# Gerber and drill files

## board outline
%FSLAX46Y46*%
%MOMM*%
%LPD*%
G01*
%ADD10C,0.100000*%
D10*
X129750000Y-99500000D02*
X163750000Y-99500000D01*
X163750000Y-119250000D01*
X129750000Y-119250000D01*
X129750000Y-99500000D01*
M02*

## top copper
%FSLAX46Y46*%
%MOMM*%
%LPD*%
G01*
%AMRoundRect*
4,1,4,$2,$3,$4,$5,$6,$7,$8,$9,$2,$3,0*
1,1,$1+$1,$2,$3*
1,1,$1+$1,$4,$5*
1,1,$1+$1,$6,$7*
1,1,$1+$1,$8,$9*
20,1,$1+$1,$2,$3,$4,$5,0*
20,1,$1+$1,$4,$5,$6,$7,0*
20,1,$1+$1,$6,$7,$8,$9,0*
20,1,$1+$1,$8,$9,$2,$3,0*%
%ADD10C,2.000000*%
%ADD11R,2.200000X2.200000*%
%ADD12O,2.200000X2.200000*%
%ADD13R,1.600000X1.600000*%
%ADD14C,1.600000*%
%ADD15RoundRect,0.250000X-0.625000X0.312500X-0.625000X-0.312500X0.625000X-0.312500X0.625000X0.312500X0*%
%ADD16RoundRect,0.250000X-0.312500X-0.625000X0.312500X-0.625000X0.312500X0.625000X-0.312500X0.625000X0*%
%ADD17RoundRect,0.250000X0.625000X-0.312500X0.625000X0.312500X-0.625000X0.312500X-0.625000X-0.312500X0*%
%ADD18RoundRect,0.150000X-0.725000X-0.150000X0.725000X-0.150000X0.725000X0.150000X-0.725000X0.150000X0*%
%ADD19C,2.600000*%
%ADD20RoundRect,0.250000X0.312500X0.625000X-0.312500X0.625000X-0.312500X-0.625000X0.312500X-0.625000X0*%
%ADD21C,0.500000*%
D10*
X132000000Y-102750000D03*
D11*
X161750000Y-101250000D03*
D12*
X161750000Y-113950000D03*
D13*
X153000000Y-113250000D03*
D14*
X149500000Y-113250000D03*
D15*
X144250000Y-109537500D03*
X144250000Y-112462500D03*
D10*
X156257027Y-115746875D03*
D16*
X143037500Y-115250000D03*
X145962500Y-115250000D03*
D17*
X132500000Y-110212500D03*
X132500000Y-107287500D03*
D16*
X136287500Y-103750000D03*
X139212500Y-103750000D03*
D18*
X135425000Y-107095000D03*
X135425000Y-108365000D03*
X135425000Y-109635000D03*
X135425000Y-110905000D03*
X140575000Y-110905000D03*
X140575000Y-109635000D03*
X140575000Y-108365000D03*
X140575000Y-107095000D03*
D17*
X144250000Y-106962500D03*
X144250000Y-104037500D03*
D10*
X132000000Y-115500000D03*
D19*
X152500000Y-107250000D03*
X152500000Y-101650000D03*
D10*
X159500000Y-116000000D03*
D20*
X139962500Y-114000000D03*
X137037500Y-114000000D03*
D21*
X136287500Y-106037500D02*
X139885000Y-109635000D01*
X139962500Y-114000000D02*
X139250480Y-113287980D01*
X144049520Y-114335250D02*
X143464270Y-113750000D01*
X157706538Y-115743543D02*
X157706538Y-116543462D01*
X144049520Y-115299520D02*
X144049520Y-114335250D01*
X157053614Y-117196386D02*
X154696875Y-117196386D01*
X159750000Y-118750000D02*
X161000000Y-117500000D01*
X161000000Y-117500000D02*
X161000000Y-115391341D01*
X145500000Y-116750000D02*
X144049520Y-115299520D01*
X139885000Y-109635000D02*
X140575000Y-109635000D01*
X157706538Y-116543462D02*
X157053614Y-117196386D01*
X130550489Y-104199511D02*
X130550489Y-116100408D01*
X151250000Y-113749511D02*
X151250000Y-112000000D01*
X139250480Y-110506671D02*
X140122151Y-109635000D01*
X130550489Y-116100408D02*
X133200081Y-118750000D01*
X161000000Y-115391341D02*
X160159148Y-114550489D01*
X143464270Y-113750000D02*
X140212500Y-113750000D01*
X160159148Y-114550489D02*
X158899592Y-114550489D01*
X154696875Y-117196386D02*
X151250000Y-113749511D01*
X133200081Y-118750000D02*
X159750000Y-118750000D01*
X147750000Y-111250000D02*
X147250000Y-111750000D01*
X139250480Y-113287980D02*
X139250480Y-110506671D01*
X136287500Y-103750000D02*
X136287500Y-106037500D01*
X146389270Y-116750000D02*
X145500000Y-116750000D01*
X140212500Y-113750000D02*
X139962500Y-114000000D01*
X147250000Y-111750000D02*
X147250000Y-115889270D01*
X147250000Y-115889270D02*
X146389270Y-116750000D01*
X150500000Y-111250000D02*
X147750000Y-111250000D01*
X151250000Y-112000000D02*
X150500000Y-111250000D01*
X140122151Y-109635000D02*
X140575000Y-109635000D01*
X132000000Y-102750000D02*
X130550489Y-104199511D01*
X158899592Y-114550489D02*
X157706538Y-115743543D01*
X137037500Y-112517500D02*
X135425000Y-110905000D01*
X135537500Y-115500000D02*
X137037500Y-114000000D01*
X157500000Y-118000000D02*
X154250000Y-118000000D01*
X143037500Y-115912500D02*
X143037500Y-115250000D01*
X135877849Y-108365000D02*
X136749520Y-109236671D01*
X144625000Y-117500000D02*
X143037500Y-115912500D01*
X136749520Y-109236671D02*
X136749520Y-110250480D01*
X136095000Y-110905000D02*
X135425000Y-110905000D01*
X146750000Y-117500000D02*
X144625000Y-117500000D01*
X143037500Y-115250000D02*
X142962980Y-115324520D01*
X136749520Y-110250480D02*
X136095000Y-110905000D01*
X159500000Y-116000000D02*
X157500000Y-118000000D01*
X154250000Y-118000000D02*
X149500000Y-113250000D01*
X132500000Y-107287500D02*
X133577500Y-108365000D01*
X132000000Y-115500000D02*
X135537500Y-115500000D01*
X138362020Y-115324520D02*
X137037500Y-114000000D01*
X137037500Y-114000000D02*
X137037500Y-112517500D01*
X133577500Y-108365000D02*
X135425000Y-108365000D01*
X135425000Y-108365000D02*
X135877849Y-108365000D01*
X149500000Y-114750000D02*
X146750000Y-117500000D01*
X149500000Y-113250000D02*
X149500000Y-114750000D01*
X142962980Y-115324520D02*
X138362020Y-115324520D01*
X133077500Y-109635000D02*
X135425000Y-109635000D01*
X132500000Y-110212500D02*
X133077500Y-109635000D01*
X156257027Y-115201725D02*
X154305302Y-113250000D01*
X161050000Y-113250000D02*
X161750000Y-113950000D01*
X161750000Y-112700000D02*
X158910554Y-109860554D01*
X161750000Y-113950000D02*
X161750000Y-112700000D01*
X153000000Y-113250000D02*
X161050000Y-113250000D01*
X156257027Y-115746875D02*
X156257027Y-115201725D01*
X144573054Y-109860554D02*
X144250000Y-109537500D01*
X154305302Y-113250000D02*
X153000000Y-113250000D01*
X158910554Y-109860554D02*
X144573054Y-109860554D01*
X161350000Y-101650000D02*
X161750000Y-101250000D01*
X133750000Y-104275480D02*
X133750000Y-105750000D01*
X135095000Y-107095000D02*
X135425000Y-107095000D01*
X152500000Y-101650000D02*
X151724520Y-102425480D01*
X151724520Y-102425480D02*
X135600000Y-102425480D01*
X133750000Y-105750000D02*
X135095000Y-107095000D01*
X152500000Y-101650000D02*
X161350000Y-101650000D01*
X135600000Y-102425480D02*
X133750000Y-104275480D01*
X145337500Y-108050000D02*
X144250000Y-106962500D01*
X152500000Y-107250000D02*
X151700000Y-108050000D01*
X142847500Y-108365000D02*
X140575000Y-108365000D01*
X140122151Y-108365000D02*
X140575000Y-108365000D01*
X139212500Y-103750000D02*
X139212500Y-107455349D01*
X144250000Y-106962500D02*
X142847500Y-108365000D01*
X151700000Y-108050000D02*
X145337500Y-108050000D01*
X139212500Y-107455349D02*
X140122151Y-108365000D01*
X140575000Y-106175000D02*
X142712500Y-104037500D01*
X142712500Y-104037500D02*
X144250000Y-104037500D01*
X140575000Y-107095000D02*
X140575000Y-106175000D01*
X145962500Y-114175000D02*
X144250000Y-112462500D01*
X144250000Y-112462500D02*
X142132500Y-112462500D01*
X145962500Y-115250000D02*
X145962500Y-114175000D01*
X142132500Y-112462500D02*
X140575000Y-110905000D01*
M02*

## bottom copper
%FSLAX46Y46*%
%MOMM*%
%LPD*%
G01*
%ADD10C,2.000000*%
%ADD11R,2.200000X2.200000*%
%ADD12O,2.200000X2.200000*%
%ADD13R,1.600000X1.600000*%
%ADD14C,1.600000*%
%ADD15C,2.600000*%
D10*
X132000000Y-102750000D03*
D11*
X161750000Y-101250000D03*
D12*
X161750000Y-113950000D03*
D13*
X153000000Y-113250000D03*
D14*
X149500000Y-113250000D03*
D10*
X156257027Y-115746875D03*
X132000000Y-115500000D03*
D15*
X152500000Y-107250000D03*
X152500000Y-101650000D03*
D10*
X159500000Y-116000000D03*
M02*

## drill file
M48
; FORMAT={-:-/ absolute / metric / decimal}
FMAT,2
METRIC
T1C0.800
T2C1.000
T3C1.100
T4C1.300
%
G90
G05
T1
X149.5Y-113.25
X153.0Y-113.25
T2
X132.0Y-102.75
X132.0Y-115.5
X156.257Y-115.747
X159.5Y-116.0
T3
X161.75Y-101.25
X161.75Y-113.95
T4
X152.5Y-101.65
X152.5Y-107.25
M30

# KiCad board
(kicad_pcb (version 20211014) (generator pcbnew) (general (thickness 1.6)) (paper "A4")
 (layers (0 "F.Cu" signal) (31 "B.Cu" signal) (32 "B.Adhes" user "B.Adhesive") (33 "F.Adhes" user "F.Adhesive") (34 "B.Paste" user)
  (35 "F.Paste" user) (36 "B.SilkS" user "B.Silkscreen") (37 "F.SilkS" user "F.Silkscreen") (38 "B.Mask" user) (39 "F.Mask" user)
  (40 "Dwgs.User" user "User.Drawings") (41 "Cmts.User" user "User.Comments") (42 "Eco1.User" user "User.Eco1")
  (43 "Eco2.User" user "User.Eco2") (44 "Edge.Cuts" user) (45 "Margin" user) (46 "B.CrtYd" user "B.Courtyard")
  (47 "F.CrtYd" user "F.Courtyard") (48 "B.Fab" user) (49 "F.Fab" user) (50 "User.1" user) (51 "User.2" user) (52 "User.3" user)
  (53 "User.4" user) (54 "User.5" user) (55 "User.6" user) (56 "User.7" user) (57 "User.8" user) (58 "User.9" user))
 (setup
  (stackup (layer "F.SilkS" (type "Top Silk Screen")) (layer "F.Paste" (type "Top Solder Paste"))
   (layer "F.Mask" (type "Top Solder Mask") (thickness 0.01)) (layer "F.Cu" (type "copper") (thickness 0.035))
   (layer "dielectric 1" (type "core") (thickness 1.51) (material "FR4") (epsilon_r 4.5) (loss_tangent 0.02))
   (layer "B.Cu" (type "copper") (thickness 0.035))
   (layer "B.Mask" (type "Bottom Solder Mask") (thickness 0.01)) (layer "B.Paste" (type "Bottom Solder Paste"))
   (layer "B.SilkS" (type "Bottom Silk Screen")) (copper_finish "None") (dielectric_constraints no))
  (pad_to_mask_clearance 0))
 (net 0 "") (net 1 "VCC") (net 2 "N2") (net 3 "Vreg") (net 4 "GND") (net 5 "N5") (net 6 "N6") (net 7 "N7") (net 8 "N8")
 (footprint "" (layer "F.Cu") (at 132 102.75)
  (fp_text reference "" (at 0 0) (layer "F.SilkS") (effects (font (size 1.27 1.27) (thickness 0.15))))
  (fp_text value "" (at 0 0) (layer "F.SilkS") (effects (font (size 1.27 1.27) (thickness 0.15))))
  (pad "1" thru_hole circle (at 0 0) (size 2 2) (drill 1) (layers *.Cu *.Mask) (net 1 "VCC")))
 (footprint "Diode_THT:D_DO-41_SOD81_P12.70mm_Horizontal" (layer "F.Cu") (at 161.75 101.25 -90)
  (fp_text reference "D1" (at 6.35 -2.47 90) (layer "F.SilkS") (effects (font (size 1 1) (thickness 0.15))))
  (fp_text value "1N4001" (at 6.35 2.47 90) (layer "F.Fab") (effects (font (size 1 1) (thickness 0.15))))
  (pad "1" thru_hole rect (at 0 0 270) (size 2.2 2.2) (drill 1.1) (layers *.Cu *.Mask) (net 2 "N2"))
  (pad "2" thru_hole oval (at 12.7 0 270) (size 2.2 2.2) (drill 1.1) (layers *.Cu *.Mask) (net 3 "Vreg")))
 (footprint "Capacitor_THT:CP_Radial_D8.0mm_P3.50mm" (layer "F.Cu") (at 153 113.25 180)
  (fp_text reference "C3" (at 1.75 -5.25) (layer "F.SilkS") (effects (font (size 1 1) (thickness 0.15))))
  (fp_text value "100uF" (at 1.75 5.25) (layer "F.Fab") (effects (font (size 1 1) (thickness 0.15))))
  (pad "1" thru_hole rect (at 0 0 180) (size 1.6 1.6) (drill 0.8) (layers *.Cu *.Mask) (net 3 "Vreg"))
  (pad "2" thru_hole circle (at 3.5 0 180) (size 1.6 1.6) (drill 0.8) (layers *.Cu *.Mask) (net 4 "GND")))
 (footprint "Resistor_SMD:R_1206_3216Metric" (layer "F.Cu") (at 144.25 111 -90)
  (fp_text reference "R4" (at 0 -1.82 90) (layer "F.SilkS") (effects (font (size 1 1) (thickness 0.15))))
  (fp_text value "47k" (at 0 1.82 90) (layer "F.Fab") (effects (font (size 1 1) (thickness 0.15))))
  (pad "1" smd roundrect (at -1.4625 0 270) (size 1.125 1.75) (layers "F.Cu" "F.Paste" "F.Mask") (roundrect_rratio 0.2222222222)
   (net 3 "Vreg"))
  (pad "2" smd roundrect (at 1.4625 0 270) (size 1.125 1.75) (layers "F.Cu" "F.Paste" "F.Mask") (roundrect_rratio 0.2222222222) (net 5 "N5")))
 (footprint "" (layer "F.Cu") (at 156.257027 115.746875)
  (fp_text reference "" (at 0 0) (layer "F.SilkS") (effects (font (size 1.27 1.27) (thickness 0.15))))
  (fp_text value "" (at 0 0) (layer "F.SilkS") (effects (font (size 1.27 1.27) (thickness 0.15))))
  (pad "1" thru_hole circle (at 0 0) (size 2 2) (drill 1) (layers *.Cu *.Mask) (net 3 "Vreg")))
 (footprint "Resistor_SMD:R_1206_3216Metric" (layer "F.Cu") (at 144.5 115.25)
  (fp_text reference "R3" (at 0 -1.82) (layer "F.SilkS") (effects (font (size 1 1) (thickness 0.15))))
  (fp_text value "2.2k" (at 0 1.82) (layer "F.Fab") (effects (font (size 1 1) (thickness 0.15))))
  (pad "1" smd roundrect (at -1.4625 0) (size 1.125 1.75) (layers "F.Cu" "F.Paste" "F.Mask") (roundrect_rratio 0.2222222222) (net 4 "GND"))
  (pad "2" smd roundrect (at 1.4625 0) (size 1.125 1.75) (layers "F.Cu" "F.Paste" "F.Mask") (roundrect_rratio 0.2222222222) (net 5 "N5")))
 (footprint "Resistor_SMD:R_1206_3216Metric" (layer "F.Cu") (at 132.5 108.75 90)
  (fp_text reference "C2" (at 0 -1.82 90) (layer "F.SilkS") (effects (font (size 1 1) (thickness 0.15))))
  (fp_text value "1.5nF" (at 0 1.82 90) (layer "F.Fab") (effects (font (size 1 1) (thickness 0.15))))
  (pad "1" smd roundrect (at -1.4625 0 90) (size 1.125 1.75) (layers "F.Cu" "F.Paste" "F.Mask") (roundrect_rratio 0.2222222222) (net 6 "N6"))
  (pad "2" smd roundrect (at 1.4625 0 90) (size 1.125 1.75) (layers "F.Cu" "F.Paste" "F.Mask") (roundrect_rratio 0.2222222222) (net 4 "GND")))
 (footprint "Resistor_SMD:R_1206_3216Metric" (layer "F.Cu") (at 137.75 103.75)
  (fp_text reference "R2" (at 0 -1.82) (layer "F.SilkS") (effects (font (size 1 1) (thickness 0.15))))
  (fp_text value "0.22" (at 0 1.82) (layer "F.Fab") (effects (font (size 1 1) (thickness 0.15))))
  (pad "1" smd roundrect (at -1.4625 0) (size 1.125 1.75) (layers "F.Cu" "F.Paste" "F.Mask") (roundrect_rratio 0.2222222222) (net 1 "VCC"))
  (pad "2" smd roundrect (at 1.4625 0) (size 1.125 1.75) (layers "F.Cu" "F.Paste" "F.Mask") (roundrect_rratio 0.2222222222) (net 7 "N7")))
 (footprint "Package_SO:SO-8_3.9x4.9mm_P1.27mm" (layer "F.Cu") (at 138 109)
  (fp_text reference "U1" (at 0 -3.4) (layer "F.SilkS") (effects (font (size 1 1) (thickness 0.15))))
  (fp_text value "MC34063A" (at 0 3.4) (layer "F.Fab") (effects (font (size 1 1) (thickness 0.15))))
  (pad "1" smd roundrect (at -2.575 -1.905) (size 1.75 0.6) (layers "F.Cu" "F.Paste" "F.Mask") (roundrect_rratio 0.25) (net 2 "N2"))
  (pad "2" smd roundrect (at -2.575 -0.635) (size 1.75 0.6) (layers "F.Cu" "F.Paste" "F.Mask") (roundrect_rratio 0.25) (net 4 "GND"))
  (pad "3" smd roundrect (at -2.575 0.635) (size 1.75 0.6) (layers "F.Cu" "F.Paste" "F.Mask") (roundrect_rratio 0.25) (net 6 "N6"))
  (pad "4" smd roundrect (at -2.575 1.905) (size 1.75 0.6) (layers "F.Cu" "F.Paste" "F.Mask") (roundrect_rratio 0.25) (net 4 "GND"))
  (pad "5" smd roundrect (at 2.575 1.905) (size 1.75 0.6) (layers "F.Cu" "F.Paste" "F.Mask") (roundrect_rratio 0.25) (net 5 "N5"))
  (pad "6" smd roundrect (at 2.575 0.635) (size 1.75 0.6) (layers "F.Cu" "F.Paste" "F.Mask") (roundrect_rratio 0.25) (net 1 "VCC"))
  (pad "7" smd roundrect (at 2.575 -0.635) (size 1.75 0.6) (layers "F.Cu" "F.Paste" "F.Mask") (roundrect_rratio 0.25) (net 7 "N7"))
  (pad "8" smd roundrect (at 2.575 -1.905) (size 1.75 0.6) (layers "F.Cu" "F.Paste" "F.Mask") (roundrect_rratio 0.25) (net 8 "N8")))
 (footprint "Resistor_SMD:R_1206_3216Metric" (layer "F.Cu") (at 144.25 105.5 90)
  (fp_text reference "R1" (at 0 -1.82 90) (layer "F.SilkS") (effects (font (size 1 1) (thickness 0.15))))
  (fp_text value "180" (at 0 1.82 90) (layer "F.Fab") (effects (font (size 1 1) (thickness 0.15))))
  (pad "1" smd roundrect (at -1.4625 0 90) (size 1.125 1.75) (layers "F.Cu" "F.Paste" "F.Mask") (roundrect_rratio 0.2222222222) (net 7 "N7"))
  (pad "2" smd roundrect (at 1.4625 0 90) (size 1.125 1.75) (layers "F.Cu" "F.Paste" "F.Mask") (roundrect_rratio 0.2222222222) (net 8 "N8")))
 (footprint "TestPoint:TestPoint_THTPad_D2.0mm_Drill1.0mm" (layer "F.Cu") (at 132 115.5)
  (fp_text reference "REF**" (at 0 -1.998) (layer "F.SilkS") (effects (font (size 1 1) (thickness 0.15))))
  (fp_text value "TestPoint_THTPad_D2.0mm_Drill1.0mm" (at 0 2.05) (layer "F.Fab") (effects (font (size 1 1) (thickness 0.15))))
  (pad "1" thru_hole circle (at 0 0) (size 2 2) (drill 1) (layers *.Cu *.Mask) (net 4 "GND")))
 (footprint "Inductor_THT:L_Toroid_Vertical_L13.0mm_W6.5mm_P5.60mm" (layer "F.Cu") (at 152.5 107.25 180)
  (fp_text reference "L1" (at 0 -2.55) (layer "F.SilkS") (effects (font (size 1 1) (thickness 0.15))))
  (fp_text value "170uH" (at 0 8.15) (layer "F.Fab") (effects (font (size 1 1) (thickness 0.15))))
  (pad "1" thru_hole circle (at 0 0 180) (size 2.6 2.6) (drill 1.3) (layers *.Cu *.Mask) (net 7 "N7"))
  (pad "2" thru_hole circle (at 0 5.6 180) (size 2.6 2.6) (drill 1.3) (layers *.Cu *.Mask) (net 2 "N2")))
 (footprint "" (layer "F.Cu") (at 159.5 116)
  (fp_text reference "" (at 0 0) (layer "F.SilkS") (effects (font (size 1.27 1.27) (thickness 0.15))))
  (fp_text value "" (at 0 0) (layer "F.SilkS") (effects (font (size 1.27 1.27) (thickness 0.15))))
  (pad "1" thru_hole circle (at 0 0) (size 2 2) (drill 1) (layers *.Cu *.Mask) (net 4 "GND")))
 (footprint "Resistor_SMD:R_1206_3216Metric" (layer "F.Cu") (at 138.5 114 180)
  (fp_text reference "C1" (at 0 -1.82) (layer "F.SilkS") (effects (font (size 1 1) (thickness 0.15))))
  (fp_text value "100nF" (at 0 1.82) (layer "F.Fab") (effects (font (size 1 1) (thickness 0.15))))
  (pad "1" smd roundrect (at -1.4625 0 180) (size 1.125 1.75) (layers "F.Cu" "F.Paste" "F.Mask") (roundrect_rratio 0.2222222222)
   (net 1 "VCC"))
  (pad "2" smd roundrect (at 1.4625 0 180) (size 1.125 1.75) (layers "F.Cu" "F.Paste" "F.Mask") (roundrect_rratio 0.2222222222)
   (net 4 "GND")))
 (gr_rect (start 129.75 99.5) (end 163.75 119.25) (layer "Edge.Cuts") (width 0.1) (fill none))
 (segment (start 136.2875 106.0375) (end 139.885 109.635) (width 0.5) (layer "F.Cu") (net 1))
 (segment (start 139.9625 114) (end 139.25048 113.28798) (width 0.5) (layer "F.Cu") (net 1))
 (segment (start 144.04952 114.33525) (end 143.46427 113.75) (width 0.5) (layer "F.Cu") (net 1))
 (segment (start 157.706538 115.743543) (end 157.706538 116.543462) (width 0.5) (layer "F.Cu") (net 1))
 (segment (start 144.04952 115.29952) (end 144.04952 114.33525) (width 0.5) (layer "F.Cu") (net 1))
 (segment (start 157.053614 117.196386) (end 154.696875 117.196386) (width 0.5) (layer "F.Cu") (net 1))
 (segment (start 159.75 118.75) (end 161 117.5) (width 0.5) (layer "F.Cu") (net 1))
 (segment (start 161 117.5) (end 161 115.391341) (width 0.5) (layer "F.Cu") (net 1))
 (segment (start 145.5 116.75) (end 144.04952 115.29952) (width 0.5) (layer "F.Cu") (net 1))
 (segment (start 139.885 109.635) (end 140.575 109.635) (width 0.5) (layer "F.Cu") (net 1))
 (segment (start 157.706538 116.543462) (end 157.053614 117.196386) (width 0.5) (layer "F.Cu") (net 1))
 (segment (start 130.550489 104.199511) (end 130.550489 116.100408) (width 0.5) (layer "F.Cu") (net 1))
 (segment (start 151.25 113.749511) (end 151.25 112) (width 0.5) (layer "F.Cu") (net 1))
 (segment (start 139.25048 110.506671) (end 140.122151 109.635) (width 0.5) (layer "F.Cu") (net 1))
 (segment (start 130.550489 116.100408) (end 133.200081 118.75) (width 0.5) (layer "F.Cu") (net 1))
 (segment (start 161 115.391341) (end 160.159148 114.550489) (width 0.5) (layer "F.Cu") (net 1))
 (segment (start 143.46427 113.75) (end 140.2125 113.75) (width 0.5) (layer "F.Cu") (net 1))
 (segment (start 160.159148 114.550489) (end 158.899592 114.550489) (width 0.5) (layer "F.Cu") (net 1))
 (segment (start 154.696875 117.196386) (end 151.25 113.749511) (width 0.5) (layer "F.Cu") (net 1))
 (segment (start 133.200081 118.75) (end 159.75 118.75) (width 0.5) (layer "F.Cu") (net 1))
 (segment (start 147.75 111.25) (end 147.25 111.75) (width 0.5) (layer "F.Cu") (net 1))
 (segment (start 139.25048 113.28798) (end 139.25048 110.506671) (width 0.5) (layer "F.Cu") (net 1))
 (segment (start 136.2875 103.75) (end 136.2875 106.0375) (width 0.5) (layer "F.Cu") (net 1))
 (segment (start 146.38927 116.75) (end 145.5 116.75) (width 0.5) (layer "F.Cu") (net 1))
 (segment (start 140.2125 113.75) (end 139.9625 114) (width 0.5) (layer "F.Cu") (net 1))
 (segment (start 147.25 111.75) (end 147.25 115.88927) (width 0.5) (layer "F.Cu") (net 1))
 (segment (start 147.25 115.88927) (end 146.38927 116.75) (width 0.5) (layer "F.Cu") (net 1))
 (segment (start 150.5 111.25) (end 147.75 111.25) (width 0.5) (layer "F.Cu") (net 1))
 (segment (start 151.25 112) (end 150.5 111.25) (width 0.5) (layer "F.Cu") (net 1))
 (segment (start 140.122151 109.635) (end 140.575 109.635) (width 0.5) (layer "F.Cu") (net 1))
 (segment (start 132 102.75) (end 130.550489 104.199511) (width 0.5) (layer "F.Cu") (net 1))
 (segment (start 158.899592 114.550489) (end 157.706538 115.743543) (width 0.5) (layer "F.Cu") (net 1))
 (segment (start 137.0375 112.5175) (end 135.425 110.905) (width 0.5) (layer "F.Cu") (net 4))
 (segment (start 135.5375 115.5) (end 137.0375 114) (width 0.5) (layer "F.Cu") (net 4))
 (segment (start 157.5 118) (end 154.25 118) (width 0.5) (layer "F.Cu") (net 4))
 (segment (start 143.0375 115.9125) (end 143.0375 115.25) (width 0.5) (layer "F.Cu") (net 4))
 (segment (start 135.877849 108.365) (end 136.74952 109.236671) (width 0.5) (layer "F.Cu") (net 4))
 (segment (start 144.625 117.5) (end 143.0375 115.9125) (width 0.5) (layer "F.Cu") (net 4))
 (segment (start 136.74952 109.236671) (end 136.74952 110.25048) (width 0.5) (layer "F.Cu") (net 4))
 (segment (start 136.095 110.905) (end 135.425 110.905) (width 0.5) (layer "F.Cu") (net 4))
 (segment (start 146.75 117.5) (end 144.625 117.5) (width 0.5) (layer "F.Cu") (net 4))
 (segment (start 143.0375 115.25) (end 142.96298 115.32452) (width 0.5) (layer "F.Cu") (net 4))
 (segment (start 136.74952 110.25048) (end 136.095 110.905) (width 0.5) (layer "F.Cu") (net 4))
 (segment (start 159.5 116) (end 157.5 118) (width 0.5) (layer "F.Cu") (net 4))
 (segment (start 154.25 118) (end 149.5 113.25) (width 0.5) (layer "F.Cu") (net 4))
 (segment (start 132.5 107.2875) (end 133.5775 108.365) (width 0.5) (layer "F.Cu") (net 4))
 (segment (start 132 115.5) (end 135.5375 115.5) (width 0.5) (layer "F.Cu") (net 4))
 (segment (start 138.36202 115.32452) (end 137.0375 114) (width 0.5) (layer "F.Cu") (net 4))
 (segment (start 137.0375 114) (end 137.0375 112.5175) (width 0.5) (layer "F.Cu") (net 4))
 (segment (start 133.5775 108.365) (end 135.425 108.365) (width 0.5) (layer "F.Cu") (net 4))
 (segment (start 135.425 108.365) (end 135.877849 108.365) (width 0.5) (layer "F.Cu") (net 4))
 (segment (start 149.5 114.75) (end 146.75 117.5) (width 0.5) (layer "F.Cu") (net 4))
 (segment (start 149.5 113.25) (end 149.5 114.75) (width 0.5) (layer "F.Cu") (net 4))
 (segment (start 142.96298 115.32452) (end 138.36202 115.32452) (width 0.5) (layer "F.Cu") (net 4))
 (segment (start 133.0775 109.635) (end 135.425 109.635) (width 0.5) (layer "F.Cu") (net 6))
 (segment (start 132.5 110.2125) (end 133.0775 109.635) (width 0.5) (layer "F.Cu") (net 6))
 (segment (start 156.257027 115.201725) (end 154.305302 113.25) (width 0.5) (layer "F.Cu") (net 3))
 (segment (start 161.05 113.25) (end 161.75 113.95) (width 0.5) (layer "F.Cu") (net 3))
 (segment (start 161.75 112.7) (end 158.910554 109.860554) (width 0.5) (layer "F.Cu") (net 3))
 (segment (start 161.75 113.95) (end 161.75 112.7) (width 0.5) (layer "F.Cu") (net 3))
 (segment (start 153 113.25) (end 161.05 113.25) (width 0.5) (layer "F.Cu") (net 3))
 (segment (start 156.257027 115.746875) (end 156.257027 115.201725) (width 0.5) (layer "F.Cu") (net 3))
 (segment (start 144.573054 109.860554) (end 144.25 109.5375) (width 0.5) (layer "F.Cu") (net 3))
 (segment (start 154.305302 113.25) (end 153 113.25) (width 0.5) (layer "F.Cu") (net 3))
 (segment (start 158.910554 109.860554) (end 144.573054 109.860554) (width 0.5) (layer "F.Cu") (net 3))
 (segment (start 161.35 101.65) (end 161.75 101.25) (width 0.5) (layer "F.Cu") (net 2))
 (segment (start 133.75 104.27548) (end 133.75 105.75) (width 0.5) (layer "F.Cu") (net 2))
 (segment (start 135.095 107.095) (end 135.425 107.095) (width 0.5) (layer "F.Cu") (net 2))
 (segment (start 152.5 101.65) (end 151.72452 102.42548) (width 0.5) (layer "F.Cu") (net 2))
 (segment (start 151.72452 102.42548) (end 135.6 102.42548) (width 0.5) (layer "F.Cu") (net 2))
 (segment (start 133.75 105.75) (end 135.095 107.095) (width 0.5) (layer "F.Cu") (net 2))
 (segment (start 152.5 101.65) (end 161.35 101.65) (width 0.5) (layer "F.Cu") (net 2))
 (segment (start 135.6 102.42548) (end 133.75 104.27548) (width 0.5) (layer "F.Cu") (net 2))
 (segment (start 145.3375 108.05) (end 144.25 106.9625) (width 0.5) (layer "F.Cu") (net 7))
 (segment (start 152.5 107.25) (end 151.7 108.05) (width 0.5) (layer "F.Cu") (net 7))
 (segment (start 142.8475 108.365) (end 140.575 108.365) (width 0.5) (layer "F.Cu") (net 7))
 (segment (start 140.122151 108.365) (end 140.575 108.365) (width 0.5) (layer "F.Cu") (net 7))
 (segment (start 139.2125 103.75) (end 139.2125 107.455349) (width 0.5) (layer "F.Cu") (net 7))
 (segment (start 144.25 106.9625) (end 142.8475 108.365) (width 0.5) (layer "F.Cu") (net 7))
 (segment (start 151.7 108.05) (end 145.3375 108.05) (width 0.5) (layer "F.Cu") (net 7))
 (segment (start 139.2125 107.455349) (end 140.122151 108.365) (width 0.5) (layer "F.Cu") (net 7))
 (segment (start 140.575 106.175) (end 142.7125 104.0375) (width 0.5) (layer "F.Cu") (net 8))
 (segment (start 142.7125 104.0375) (end 144.25 104.0375) (width 0.5) (layer "F.Cu") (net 8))
 (segment (start 140.575 107.095) (end 140.575 106.175) (width 0.5) (layer "F.Cu") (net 8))
 (segment (start 145.9625 114.175) (end 144.25 112.4625) (width 0.5) (layer "F.Cu") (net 5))
 (segment (start 144.25 112.4625) (end 142.1325 112.4625) (width 0.5) (layer "F.Cu") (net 5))
 (segment (start 145.9625 115.25) (end 145.9625 114.175) (width 0.5) (layer "F.Cu") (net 5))
 (segment (start 142.1325 112.4625) (end 140.575 110.905) (width 0.5) (layer "F.Cu") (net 5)))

